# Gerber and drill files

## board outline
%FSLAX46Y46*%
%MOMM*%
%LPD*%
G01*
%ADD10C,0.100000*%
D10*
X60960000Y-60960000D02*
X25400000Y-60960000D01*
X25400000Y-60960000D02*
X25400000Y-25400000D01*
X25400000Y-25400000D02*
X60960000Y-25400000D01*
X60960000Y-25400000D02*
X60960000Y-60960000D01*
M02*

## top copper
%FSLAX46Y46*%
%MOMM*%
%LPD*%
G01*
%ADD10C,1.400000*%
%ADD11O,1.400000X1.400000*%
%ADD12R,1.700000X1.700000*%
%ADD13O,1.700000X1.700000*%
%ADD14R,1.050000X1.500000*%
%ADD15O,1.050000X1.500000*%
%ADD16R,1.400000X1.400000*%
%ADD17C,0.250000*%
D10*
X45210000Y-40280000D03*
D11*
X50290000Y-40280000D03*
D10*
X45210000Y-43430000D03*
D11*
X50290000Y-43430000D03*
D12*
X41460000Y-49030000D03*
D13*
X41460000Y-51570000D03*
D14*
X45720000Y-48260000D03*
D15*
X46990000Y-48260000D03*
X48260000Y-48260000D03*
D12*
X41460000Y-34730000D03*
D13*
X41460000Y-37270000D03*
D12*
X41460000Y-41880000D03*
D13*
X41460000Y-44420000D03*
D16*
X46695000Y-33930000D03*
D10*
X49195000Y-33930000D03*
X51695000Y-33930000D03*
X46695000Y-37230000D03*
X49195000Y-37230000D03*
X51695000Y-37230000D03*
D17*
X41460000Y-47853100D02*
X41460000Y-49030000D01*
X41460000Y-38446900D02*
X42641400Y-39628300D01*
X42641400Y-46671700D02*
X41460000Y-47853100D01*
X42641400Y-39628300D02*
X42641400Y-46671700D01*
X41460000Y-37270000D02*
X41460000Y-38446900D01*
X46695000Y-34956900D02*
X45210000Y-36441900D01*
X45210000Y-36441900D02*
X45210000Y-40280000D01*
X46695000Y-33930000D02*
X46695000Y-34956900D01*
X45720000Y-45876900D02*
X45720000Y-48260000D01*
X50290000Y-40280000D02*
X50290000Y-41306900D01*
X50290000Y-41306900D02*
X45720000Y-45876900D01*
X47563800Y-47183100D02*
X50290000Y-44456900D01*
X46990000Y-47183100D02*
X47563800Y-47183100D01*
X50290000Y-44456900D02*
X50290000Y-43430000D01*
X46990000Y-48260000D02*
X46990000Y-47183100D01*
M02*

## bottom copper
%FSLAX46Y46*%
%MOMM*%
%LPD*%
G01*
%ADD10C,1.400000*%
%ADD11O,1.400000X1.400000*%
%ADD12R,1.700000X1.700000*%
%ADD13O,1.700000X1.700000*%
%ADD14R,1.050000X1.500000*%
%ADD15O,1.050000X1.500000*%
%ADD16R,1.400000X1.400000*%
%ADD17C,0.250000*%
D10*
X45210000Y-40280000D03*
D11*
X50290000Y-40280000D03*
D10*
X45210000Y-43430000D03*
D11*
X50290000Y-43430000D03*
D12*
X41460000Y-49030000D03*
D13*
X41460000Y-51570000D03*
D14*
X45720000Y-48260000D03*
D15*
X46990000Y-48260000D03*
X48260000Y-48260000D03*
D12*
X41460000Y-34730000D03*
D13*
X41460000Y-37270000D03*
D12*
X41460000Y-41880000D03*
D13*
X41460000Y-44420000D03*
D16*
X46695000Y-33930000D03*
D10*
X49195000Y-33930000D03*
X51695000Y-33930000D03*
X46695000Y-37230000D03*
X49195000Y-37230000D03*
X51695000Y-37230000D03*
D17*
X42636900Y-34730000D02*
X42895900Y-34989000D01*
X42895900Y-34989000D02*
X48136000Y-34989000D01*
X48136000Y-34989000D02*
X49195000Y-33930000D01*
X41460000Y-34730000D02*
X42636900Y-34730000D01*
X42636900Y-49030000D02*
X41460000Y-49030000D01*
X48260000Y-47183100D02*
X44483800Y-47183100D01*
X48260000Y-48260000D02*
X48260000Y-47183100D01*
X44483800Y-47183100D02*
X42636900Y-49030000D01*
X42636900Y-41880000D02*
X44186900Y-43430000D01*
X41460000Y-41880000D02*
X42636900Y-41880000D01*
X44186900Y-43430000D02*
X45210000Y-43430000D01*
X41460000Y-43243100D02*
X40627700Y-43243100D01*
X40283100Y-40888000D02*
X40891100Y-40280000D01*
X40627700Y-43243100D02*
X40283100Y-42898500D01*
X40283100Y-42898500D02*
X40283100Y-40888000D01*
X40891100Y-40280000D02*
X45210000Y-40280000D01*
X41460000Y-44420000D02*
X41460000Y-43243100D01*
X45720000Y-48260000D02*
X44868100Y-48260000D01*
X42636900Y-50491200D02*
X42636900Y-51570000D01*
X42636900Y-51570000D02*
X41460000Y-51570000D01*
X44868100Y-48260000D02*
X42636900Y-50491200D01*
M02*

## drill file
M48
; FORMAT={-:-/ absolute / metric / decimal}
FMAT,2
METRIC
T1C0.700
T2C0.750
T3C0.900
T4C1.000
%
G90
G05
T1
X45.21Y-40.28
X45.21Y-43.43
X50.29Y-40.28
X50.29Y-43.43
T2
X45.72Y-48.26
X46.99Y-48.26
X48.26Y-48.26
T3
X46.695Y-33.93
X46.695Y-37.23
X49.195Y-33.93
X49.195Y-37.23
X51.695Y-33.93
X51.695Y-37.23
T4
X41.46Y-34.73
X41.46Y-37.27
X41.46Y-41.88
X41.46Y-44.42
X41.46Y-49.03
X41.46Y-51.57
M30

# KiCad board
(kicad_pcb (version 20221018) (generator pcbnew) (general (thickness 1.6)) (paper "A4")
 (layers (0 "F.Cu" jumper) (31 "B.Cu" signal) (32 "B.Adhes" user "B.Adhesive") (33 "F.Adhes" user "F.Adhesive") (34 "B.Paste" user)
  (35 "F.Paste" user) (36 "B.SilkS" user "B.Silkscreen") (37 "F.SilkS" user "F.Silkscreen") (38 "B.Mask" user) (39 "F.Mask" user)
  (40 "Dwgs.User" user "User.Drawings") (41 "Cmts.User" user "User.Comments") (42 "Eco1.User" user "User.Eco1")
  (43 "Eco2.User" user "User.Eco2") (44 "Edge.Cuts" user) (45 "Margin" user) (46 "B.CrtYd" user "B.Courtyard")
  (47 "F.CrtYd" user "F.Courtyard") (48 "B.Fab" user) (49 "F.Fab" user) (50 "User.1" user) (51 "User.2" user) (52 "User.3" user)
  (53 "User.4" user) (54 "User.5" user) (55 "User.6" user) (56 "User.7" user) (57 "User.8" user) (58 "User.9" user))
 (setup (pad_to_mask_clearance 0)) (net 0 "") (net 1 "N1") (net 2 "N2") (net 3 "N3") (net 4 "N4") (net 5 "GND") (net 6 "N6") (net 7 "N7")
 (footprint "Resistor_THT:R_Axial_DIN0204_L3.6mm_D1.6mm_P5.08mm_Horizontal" (layer "F.Cu") (at 45.21 40.28)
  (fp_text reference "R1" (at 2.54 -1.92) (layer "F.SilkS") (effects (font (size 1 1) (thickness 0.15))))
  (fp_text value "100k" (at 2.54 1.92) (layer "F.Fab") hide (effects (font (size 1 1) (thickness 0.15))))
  (pad "1" thru_hole circle (at 0 0) (size 1.4 1.4) (drill 0.7) (layers "*.Cu" "*.Mask") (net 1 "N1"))
  (pad "2" thru_hole oval (at 5.08 0) (size 1.4 1.4) (drill 0.7) (layers "*.Cu" "*.Mask") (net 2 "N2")))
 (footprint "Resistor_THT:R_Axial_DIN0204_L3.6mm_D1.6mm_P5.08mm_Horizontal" (layer "F.Cu") (at 45.21 43.43)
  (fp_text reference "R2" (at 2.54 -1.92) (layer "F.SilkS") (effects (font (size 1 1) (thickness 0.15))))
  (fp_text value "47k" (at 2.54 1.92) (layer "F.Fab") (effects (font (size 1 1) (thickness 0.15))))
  (pad "1" thru_hole circle (at 0 0) (size 1.4 1.4) (drill 0.7) (layers "*.Cu" "*.Mask") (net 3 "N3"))
  (pad "2" thru_hole oval (at 5.08 0) (size 1.4 1.4) (drill 0.7) (layers "*.Cu" "*.Mask") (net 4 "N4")))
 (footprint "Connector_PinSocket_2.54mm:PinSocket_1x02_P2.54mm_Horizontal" (layer "F.Cu") (at 41.46 49.03)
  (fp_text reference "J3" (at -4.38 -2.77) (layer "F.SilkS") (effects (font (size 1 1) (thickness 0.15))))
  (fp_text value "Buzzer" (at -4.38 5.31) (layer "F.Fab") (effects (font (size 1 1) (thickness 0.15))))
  (pad "1" thru_hole rect (at 0 0) (size 1.7 1.7) (drill 1) (layers "*.Cu" "*.Mask") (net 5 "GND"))
  (pad "2" thru_hole oval (at 0 2.54) (size 1.7 1.7) (drill 1) (layers "*.Cu" "*.Mask") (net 2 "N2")))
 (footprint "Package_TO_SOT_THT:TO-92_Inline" (layer "F.Cu") (at 45.72 48.26)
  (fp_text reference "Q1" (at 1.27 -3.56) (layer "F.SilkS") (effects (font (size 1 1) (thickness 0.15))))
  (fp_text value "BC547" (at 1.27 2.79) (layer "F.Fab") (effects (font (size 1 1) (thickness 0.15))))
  (pad "1" thru_hole rect (at 0 0) (size 1.05 1.5) (drill 0.75) (layers "*.Cu" "*.Mask") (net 2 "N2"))
  (pad "2" thru_hole oval (at 1.27 0) (size 1.05 1.5) (drill 0.75) (layers "*.Cu" "*.Mask") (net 4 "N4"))
  (pad "3" thru_hole oval (at 2.54 0) (size 1.05 1.5) (drill 0.75) (layers "*.Cu" "*.Mask") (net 5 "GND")))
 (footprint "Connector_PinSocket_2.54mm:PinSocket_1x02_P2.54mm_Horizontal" (layer "F.Cu") (at 41.46 34.73)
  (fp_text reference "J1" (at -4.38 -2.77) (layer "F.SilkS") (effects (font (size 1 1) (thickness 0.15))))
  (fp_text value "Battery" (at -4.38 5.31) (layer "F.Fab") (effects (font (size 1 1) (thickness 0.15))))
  (pad "1" thru_hole rect (at 0 0) (size 1.7 1.7) (drill 1) (layers "*.Cu" "*.Mask") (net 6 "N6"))
  (pad "2" thru_hole oval (at 0 2.54) (size 1.7 1.7) (drill 1) (layers "*.Cu" "*.Mask") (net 5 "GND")))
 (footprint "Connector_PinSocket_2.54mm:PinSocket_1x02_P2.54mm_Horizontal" (layer "F.Cu") (at 41.46 41.88)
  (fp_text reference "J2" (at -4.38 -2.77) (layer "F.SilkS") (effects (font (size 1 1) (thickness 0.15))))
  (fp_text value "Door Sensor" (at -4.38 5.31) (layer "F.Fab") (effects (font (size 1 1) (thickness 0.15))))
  (pad "1" thru_hole rect (at 0 0) (size 1.7 1.7) (drill 1) (layers "*.Cu" "*.Mask") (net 3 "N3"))
  (pad "2" thru_hole oval (at 0 2.54) (size 1.7 1.7) (drill 1) (layers "*.Cu" "*.Mask") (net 1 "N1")))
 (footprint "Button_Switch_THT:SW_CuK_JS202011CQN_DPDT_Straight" (layer "F.Cu") (at 46.695 33.93)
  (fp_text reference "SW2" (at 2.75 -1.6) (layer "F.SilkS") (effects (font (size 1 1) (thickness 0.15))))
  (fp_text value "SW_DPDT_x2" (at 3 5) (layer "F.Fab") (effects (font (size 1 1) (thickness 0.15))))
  (pad "1" thru_hole rect (at 0 0) (size 1.4 1.4) (drill 0.9) (layers "*.Cu" "*.Mask") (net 1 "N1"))
  (pad "2" thru_hole circle (at 2.5 0) (size 1.4 1.4) (drill 0.9) (layers "*.Cu" "*.Mask") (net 6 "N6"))
  (pad "3" thru_hole circle (at 5 0) (size 1.4 1.4) (drill 0.9) (layers "*.Cu" "*.Mask") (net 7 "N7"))
  (pad "4" thru_hole circle (at 0 3.3) (size 1.4 1.4) (drill 0.9) (layers "*.Cu" "*.Mask"))
  (pad "5" thru_hole circle (at 2.5 3.3) (size 1.4 1.4) (drill 0.9) (layers "*.Cu" "*.Mask"))
  (pad "6" thru_hole circle (at 5 3.3) (size 1.4 1.4) (drill 0.9) (layers "*.Cu" "*.Mask")))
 (gr_line (start 60.96 60.96) (end 25.4 60.96) (stroke (width 0.1) (type default)) (layer "Edge.Cuts"))
 (gr_line (start 25.4 60.96) (end 25.4 25.4) (stroke (width 0.1) (type default)) (layer "Edge.Cuts"))
 (gr_line (start 25.4 25.4) (end 60.96 25.4) (stroke (width 0.1) (type default)) (layer "Edge.Cuts"))
 (gr_line (start 60.96 25.4) (end 60.96 60.96) (stroke (width 0.1) (type default)) (layer "Edge.Cuts"))
 (segment (start 42.6369 34.73) (end 42.8959 34.989) (width 0.25) (layer "B.Cu") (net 6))
 (segment (start 42.8959 34.989) (end 48.136 34.989) (width 0.25) (layer "B.Cu") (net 6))
 (segment (start 48.136 34.989) (end 49.195 33.93) (width 0.25) (layer "B.Cu") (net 6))
 (segment (start 41.46 34.73) (end 42.6369 34.73) (width 0.25) (layer "B.Cu") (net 6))
 (segment (start 41.46 47.8531) (end 41.46 49.03) (width 0.25) (layer "F.Cu") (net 5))
 (segment (start 41.46 38.4469) (end 42.6414 39.6283) (width 0.25) (layer "F.Cu") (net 5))
 (segment (start 42.6414 46.6717) (end 41.46 47.8531) (width 0.25) (layer "F.Cu") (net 5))
 (segment (start 42.6414 39.6283) (end 42.6414 46.6717) (width 0.25) (layer "F.Cu") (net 5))
 (segment (start 41.46 37.27) (end 41.46 38.4469) (width 0.25) (layer "F.Cu") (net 5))
 (segment (start 42.6369 49.03) (end 41.46 49.03) (width 0.25) (layer "B.Cu") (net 5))
 (segment (start 48.26 47.1831) (end 44.4838 47.1831) (width 0.25) (layer "B.Cu") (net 5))
 (segment (start 48.26 48.26) (end 48.26 47.1831) (width 0.25) (layer "B.Cu") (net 5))
 (segment (start 44.4838 47.1831) (end 42.6369 49.03) (width 0.25) (layer "B.Cu") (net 5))
 (segment (start 42.6369 41.88) (end 44.1869 43.43) (width 0.25) (layer "B.Cu") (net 3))
 (segment (start 41.46 41.88) (end 42.6369 41.88) (width 0.25) (layer "B.Cu") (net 3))
 (segment (start 44.1869 43.43) (end 45.21 43.43) (width 0.25) (layer "B.Cu") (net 3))
 (segment (start 46.695 34.9569) (end 45.21 36.4419) (width 0.25) (layer "F.Cu") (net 1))
 (segment (start 45.21 36.4419) (end 45.21 40.28) (width 0.25) (layer "F.Cu") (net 1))
 (segment (start 46.695 33.93) (end 46.695 34.9569) (width 0.25) (layer "F.Cu") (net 1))
 (segment (start 41.46 43.2431) (end 40.6277 43.2431) (width 0.25) (layer "B.Cu") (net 1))
 (segment (start 40.2831 40.888) (end 40.8911 40.28) (width 0.25) (layer "B.Cu") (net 1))
 (segment (start 40.6277 43.2431) (end 40.2831 42.8985) (width 0.25) (layer "B.Cu") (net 1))
 (segment (start 40.2831 42.8985) (end 40.2831 40.888) (width 0.25) (layer "B.Cu") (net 1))
 (segment (start 40.8911 40.28) (end 45.21 40.28) (width 0.25) (layer "B.Cu") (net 1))
 (segment (start 41.46 44.42) (end 41.46 43.2431) (width 0.25) (layer "B.Cu") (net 1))
 (segment (start 45.72 45.8769) (end 45.72 48.26) (width 0.25) (layer "F.Cu") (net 2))
 (segment (start 50.29 40.28) (end 50.29 41.3069) (width 0.25) (layer "F.Cu") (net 2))
 (segment (start 50.29 41.3069) (end 45.72 45.8769) (width 0.25) (layer "F.Cu") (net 2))
 (segment (start 45.72 48.26) (end 44.8681 48.26) (width 0.25) (layer "B.Cu") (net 2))
 (segment (start 42.6369 50.4912) (end 42.6369 51.57) (width 0.25) (layer "B.Cu") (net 2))
 (segment (start 42.6369 51.57) (end 41.46 51.57) (width 0.25) (layer "B.Cu") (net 2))
 (segment (start 44.8681 48.26) (end 42.6369 50.4912) (width 0.25) (layer "B.Cu") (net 2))
 (segment (start 47.5638 47.1831) (end 50.29 44.4569) (width 0.25) (layer "F.Cu") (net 4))
 (segment (start 46.99 47.1831) (end 47.5638 47.1831) (width 0.25) (layer "F.Cu") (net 4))
 (segment (start 50.29 44.4569) (end 50.29 43.43) (width 0.25) (layer "F.Cu") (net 4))
 (segment (start 46.99 48.26) (end 46.99 47.1831) (width 0.25) (layer "F.Cu") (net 4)))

